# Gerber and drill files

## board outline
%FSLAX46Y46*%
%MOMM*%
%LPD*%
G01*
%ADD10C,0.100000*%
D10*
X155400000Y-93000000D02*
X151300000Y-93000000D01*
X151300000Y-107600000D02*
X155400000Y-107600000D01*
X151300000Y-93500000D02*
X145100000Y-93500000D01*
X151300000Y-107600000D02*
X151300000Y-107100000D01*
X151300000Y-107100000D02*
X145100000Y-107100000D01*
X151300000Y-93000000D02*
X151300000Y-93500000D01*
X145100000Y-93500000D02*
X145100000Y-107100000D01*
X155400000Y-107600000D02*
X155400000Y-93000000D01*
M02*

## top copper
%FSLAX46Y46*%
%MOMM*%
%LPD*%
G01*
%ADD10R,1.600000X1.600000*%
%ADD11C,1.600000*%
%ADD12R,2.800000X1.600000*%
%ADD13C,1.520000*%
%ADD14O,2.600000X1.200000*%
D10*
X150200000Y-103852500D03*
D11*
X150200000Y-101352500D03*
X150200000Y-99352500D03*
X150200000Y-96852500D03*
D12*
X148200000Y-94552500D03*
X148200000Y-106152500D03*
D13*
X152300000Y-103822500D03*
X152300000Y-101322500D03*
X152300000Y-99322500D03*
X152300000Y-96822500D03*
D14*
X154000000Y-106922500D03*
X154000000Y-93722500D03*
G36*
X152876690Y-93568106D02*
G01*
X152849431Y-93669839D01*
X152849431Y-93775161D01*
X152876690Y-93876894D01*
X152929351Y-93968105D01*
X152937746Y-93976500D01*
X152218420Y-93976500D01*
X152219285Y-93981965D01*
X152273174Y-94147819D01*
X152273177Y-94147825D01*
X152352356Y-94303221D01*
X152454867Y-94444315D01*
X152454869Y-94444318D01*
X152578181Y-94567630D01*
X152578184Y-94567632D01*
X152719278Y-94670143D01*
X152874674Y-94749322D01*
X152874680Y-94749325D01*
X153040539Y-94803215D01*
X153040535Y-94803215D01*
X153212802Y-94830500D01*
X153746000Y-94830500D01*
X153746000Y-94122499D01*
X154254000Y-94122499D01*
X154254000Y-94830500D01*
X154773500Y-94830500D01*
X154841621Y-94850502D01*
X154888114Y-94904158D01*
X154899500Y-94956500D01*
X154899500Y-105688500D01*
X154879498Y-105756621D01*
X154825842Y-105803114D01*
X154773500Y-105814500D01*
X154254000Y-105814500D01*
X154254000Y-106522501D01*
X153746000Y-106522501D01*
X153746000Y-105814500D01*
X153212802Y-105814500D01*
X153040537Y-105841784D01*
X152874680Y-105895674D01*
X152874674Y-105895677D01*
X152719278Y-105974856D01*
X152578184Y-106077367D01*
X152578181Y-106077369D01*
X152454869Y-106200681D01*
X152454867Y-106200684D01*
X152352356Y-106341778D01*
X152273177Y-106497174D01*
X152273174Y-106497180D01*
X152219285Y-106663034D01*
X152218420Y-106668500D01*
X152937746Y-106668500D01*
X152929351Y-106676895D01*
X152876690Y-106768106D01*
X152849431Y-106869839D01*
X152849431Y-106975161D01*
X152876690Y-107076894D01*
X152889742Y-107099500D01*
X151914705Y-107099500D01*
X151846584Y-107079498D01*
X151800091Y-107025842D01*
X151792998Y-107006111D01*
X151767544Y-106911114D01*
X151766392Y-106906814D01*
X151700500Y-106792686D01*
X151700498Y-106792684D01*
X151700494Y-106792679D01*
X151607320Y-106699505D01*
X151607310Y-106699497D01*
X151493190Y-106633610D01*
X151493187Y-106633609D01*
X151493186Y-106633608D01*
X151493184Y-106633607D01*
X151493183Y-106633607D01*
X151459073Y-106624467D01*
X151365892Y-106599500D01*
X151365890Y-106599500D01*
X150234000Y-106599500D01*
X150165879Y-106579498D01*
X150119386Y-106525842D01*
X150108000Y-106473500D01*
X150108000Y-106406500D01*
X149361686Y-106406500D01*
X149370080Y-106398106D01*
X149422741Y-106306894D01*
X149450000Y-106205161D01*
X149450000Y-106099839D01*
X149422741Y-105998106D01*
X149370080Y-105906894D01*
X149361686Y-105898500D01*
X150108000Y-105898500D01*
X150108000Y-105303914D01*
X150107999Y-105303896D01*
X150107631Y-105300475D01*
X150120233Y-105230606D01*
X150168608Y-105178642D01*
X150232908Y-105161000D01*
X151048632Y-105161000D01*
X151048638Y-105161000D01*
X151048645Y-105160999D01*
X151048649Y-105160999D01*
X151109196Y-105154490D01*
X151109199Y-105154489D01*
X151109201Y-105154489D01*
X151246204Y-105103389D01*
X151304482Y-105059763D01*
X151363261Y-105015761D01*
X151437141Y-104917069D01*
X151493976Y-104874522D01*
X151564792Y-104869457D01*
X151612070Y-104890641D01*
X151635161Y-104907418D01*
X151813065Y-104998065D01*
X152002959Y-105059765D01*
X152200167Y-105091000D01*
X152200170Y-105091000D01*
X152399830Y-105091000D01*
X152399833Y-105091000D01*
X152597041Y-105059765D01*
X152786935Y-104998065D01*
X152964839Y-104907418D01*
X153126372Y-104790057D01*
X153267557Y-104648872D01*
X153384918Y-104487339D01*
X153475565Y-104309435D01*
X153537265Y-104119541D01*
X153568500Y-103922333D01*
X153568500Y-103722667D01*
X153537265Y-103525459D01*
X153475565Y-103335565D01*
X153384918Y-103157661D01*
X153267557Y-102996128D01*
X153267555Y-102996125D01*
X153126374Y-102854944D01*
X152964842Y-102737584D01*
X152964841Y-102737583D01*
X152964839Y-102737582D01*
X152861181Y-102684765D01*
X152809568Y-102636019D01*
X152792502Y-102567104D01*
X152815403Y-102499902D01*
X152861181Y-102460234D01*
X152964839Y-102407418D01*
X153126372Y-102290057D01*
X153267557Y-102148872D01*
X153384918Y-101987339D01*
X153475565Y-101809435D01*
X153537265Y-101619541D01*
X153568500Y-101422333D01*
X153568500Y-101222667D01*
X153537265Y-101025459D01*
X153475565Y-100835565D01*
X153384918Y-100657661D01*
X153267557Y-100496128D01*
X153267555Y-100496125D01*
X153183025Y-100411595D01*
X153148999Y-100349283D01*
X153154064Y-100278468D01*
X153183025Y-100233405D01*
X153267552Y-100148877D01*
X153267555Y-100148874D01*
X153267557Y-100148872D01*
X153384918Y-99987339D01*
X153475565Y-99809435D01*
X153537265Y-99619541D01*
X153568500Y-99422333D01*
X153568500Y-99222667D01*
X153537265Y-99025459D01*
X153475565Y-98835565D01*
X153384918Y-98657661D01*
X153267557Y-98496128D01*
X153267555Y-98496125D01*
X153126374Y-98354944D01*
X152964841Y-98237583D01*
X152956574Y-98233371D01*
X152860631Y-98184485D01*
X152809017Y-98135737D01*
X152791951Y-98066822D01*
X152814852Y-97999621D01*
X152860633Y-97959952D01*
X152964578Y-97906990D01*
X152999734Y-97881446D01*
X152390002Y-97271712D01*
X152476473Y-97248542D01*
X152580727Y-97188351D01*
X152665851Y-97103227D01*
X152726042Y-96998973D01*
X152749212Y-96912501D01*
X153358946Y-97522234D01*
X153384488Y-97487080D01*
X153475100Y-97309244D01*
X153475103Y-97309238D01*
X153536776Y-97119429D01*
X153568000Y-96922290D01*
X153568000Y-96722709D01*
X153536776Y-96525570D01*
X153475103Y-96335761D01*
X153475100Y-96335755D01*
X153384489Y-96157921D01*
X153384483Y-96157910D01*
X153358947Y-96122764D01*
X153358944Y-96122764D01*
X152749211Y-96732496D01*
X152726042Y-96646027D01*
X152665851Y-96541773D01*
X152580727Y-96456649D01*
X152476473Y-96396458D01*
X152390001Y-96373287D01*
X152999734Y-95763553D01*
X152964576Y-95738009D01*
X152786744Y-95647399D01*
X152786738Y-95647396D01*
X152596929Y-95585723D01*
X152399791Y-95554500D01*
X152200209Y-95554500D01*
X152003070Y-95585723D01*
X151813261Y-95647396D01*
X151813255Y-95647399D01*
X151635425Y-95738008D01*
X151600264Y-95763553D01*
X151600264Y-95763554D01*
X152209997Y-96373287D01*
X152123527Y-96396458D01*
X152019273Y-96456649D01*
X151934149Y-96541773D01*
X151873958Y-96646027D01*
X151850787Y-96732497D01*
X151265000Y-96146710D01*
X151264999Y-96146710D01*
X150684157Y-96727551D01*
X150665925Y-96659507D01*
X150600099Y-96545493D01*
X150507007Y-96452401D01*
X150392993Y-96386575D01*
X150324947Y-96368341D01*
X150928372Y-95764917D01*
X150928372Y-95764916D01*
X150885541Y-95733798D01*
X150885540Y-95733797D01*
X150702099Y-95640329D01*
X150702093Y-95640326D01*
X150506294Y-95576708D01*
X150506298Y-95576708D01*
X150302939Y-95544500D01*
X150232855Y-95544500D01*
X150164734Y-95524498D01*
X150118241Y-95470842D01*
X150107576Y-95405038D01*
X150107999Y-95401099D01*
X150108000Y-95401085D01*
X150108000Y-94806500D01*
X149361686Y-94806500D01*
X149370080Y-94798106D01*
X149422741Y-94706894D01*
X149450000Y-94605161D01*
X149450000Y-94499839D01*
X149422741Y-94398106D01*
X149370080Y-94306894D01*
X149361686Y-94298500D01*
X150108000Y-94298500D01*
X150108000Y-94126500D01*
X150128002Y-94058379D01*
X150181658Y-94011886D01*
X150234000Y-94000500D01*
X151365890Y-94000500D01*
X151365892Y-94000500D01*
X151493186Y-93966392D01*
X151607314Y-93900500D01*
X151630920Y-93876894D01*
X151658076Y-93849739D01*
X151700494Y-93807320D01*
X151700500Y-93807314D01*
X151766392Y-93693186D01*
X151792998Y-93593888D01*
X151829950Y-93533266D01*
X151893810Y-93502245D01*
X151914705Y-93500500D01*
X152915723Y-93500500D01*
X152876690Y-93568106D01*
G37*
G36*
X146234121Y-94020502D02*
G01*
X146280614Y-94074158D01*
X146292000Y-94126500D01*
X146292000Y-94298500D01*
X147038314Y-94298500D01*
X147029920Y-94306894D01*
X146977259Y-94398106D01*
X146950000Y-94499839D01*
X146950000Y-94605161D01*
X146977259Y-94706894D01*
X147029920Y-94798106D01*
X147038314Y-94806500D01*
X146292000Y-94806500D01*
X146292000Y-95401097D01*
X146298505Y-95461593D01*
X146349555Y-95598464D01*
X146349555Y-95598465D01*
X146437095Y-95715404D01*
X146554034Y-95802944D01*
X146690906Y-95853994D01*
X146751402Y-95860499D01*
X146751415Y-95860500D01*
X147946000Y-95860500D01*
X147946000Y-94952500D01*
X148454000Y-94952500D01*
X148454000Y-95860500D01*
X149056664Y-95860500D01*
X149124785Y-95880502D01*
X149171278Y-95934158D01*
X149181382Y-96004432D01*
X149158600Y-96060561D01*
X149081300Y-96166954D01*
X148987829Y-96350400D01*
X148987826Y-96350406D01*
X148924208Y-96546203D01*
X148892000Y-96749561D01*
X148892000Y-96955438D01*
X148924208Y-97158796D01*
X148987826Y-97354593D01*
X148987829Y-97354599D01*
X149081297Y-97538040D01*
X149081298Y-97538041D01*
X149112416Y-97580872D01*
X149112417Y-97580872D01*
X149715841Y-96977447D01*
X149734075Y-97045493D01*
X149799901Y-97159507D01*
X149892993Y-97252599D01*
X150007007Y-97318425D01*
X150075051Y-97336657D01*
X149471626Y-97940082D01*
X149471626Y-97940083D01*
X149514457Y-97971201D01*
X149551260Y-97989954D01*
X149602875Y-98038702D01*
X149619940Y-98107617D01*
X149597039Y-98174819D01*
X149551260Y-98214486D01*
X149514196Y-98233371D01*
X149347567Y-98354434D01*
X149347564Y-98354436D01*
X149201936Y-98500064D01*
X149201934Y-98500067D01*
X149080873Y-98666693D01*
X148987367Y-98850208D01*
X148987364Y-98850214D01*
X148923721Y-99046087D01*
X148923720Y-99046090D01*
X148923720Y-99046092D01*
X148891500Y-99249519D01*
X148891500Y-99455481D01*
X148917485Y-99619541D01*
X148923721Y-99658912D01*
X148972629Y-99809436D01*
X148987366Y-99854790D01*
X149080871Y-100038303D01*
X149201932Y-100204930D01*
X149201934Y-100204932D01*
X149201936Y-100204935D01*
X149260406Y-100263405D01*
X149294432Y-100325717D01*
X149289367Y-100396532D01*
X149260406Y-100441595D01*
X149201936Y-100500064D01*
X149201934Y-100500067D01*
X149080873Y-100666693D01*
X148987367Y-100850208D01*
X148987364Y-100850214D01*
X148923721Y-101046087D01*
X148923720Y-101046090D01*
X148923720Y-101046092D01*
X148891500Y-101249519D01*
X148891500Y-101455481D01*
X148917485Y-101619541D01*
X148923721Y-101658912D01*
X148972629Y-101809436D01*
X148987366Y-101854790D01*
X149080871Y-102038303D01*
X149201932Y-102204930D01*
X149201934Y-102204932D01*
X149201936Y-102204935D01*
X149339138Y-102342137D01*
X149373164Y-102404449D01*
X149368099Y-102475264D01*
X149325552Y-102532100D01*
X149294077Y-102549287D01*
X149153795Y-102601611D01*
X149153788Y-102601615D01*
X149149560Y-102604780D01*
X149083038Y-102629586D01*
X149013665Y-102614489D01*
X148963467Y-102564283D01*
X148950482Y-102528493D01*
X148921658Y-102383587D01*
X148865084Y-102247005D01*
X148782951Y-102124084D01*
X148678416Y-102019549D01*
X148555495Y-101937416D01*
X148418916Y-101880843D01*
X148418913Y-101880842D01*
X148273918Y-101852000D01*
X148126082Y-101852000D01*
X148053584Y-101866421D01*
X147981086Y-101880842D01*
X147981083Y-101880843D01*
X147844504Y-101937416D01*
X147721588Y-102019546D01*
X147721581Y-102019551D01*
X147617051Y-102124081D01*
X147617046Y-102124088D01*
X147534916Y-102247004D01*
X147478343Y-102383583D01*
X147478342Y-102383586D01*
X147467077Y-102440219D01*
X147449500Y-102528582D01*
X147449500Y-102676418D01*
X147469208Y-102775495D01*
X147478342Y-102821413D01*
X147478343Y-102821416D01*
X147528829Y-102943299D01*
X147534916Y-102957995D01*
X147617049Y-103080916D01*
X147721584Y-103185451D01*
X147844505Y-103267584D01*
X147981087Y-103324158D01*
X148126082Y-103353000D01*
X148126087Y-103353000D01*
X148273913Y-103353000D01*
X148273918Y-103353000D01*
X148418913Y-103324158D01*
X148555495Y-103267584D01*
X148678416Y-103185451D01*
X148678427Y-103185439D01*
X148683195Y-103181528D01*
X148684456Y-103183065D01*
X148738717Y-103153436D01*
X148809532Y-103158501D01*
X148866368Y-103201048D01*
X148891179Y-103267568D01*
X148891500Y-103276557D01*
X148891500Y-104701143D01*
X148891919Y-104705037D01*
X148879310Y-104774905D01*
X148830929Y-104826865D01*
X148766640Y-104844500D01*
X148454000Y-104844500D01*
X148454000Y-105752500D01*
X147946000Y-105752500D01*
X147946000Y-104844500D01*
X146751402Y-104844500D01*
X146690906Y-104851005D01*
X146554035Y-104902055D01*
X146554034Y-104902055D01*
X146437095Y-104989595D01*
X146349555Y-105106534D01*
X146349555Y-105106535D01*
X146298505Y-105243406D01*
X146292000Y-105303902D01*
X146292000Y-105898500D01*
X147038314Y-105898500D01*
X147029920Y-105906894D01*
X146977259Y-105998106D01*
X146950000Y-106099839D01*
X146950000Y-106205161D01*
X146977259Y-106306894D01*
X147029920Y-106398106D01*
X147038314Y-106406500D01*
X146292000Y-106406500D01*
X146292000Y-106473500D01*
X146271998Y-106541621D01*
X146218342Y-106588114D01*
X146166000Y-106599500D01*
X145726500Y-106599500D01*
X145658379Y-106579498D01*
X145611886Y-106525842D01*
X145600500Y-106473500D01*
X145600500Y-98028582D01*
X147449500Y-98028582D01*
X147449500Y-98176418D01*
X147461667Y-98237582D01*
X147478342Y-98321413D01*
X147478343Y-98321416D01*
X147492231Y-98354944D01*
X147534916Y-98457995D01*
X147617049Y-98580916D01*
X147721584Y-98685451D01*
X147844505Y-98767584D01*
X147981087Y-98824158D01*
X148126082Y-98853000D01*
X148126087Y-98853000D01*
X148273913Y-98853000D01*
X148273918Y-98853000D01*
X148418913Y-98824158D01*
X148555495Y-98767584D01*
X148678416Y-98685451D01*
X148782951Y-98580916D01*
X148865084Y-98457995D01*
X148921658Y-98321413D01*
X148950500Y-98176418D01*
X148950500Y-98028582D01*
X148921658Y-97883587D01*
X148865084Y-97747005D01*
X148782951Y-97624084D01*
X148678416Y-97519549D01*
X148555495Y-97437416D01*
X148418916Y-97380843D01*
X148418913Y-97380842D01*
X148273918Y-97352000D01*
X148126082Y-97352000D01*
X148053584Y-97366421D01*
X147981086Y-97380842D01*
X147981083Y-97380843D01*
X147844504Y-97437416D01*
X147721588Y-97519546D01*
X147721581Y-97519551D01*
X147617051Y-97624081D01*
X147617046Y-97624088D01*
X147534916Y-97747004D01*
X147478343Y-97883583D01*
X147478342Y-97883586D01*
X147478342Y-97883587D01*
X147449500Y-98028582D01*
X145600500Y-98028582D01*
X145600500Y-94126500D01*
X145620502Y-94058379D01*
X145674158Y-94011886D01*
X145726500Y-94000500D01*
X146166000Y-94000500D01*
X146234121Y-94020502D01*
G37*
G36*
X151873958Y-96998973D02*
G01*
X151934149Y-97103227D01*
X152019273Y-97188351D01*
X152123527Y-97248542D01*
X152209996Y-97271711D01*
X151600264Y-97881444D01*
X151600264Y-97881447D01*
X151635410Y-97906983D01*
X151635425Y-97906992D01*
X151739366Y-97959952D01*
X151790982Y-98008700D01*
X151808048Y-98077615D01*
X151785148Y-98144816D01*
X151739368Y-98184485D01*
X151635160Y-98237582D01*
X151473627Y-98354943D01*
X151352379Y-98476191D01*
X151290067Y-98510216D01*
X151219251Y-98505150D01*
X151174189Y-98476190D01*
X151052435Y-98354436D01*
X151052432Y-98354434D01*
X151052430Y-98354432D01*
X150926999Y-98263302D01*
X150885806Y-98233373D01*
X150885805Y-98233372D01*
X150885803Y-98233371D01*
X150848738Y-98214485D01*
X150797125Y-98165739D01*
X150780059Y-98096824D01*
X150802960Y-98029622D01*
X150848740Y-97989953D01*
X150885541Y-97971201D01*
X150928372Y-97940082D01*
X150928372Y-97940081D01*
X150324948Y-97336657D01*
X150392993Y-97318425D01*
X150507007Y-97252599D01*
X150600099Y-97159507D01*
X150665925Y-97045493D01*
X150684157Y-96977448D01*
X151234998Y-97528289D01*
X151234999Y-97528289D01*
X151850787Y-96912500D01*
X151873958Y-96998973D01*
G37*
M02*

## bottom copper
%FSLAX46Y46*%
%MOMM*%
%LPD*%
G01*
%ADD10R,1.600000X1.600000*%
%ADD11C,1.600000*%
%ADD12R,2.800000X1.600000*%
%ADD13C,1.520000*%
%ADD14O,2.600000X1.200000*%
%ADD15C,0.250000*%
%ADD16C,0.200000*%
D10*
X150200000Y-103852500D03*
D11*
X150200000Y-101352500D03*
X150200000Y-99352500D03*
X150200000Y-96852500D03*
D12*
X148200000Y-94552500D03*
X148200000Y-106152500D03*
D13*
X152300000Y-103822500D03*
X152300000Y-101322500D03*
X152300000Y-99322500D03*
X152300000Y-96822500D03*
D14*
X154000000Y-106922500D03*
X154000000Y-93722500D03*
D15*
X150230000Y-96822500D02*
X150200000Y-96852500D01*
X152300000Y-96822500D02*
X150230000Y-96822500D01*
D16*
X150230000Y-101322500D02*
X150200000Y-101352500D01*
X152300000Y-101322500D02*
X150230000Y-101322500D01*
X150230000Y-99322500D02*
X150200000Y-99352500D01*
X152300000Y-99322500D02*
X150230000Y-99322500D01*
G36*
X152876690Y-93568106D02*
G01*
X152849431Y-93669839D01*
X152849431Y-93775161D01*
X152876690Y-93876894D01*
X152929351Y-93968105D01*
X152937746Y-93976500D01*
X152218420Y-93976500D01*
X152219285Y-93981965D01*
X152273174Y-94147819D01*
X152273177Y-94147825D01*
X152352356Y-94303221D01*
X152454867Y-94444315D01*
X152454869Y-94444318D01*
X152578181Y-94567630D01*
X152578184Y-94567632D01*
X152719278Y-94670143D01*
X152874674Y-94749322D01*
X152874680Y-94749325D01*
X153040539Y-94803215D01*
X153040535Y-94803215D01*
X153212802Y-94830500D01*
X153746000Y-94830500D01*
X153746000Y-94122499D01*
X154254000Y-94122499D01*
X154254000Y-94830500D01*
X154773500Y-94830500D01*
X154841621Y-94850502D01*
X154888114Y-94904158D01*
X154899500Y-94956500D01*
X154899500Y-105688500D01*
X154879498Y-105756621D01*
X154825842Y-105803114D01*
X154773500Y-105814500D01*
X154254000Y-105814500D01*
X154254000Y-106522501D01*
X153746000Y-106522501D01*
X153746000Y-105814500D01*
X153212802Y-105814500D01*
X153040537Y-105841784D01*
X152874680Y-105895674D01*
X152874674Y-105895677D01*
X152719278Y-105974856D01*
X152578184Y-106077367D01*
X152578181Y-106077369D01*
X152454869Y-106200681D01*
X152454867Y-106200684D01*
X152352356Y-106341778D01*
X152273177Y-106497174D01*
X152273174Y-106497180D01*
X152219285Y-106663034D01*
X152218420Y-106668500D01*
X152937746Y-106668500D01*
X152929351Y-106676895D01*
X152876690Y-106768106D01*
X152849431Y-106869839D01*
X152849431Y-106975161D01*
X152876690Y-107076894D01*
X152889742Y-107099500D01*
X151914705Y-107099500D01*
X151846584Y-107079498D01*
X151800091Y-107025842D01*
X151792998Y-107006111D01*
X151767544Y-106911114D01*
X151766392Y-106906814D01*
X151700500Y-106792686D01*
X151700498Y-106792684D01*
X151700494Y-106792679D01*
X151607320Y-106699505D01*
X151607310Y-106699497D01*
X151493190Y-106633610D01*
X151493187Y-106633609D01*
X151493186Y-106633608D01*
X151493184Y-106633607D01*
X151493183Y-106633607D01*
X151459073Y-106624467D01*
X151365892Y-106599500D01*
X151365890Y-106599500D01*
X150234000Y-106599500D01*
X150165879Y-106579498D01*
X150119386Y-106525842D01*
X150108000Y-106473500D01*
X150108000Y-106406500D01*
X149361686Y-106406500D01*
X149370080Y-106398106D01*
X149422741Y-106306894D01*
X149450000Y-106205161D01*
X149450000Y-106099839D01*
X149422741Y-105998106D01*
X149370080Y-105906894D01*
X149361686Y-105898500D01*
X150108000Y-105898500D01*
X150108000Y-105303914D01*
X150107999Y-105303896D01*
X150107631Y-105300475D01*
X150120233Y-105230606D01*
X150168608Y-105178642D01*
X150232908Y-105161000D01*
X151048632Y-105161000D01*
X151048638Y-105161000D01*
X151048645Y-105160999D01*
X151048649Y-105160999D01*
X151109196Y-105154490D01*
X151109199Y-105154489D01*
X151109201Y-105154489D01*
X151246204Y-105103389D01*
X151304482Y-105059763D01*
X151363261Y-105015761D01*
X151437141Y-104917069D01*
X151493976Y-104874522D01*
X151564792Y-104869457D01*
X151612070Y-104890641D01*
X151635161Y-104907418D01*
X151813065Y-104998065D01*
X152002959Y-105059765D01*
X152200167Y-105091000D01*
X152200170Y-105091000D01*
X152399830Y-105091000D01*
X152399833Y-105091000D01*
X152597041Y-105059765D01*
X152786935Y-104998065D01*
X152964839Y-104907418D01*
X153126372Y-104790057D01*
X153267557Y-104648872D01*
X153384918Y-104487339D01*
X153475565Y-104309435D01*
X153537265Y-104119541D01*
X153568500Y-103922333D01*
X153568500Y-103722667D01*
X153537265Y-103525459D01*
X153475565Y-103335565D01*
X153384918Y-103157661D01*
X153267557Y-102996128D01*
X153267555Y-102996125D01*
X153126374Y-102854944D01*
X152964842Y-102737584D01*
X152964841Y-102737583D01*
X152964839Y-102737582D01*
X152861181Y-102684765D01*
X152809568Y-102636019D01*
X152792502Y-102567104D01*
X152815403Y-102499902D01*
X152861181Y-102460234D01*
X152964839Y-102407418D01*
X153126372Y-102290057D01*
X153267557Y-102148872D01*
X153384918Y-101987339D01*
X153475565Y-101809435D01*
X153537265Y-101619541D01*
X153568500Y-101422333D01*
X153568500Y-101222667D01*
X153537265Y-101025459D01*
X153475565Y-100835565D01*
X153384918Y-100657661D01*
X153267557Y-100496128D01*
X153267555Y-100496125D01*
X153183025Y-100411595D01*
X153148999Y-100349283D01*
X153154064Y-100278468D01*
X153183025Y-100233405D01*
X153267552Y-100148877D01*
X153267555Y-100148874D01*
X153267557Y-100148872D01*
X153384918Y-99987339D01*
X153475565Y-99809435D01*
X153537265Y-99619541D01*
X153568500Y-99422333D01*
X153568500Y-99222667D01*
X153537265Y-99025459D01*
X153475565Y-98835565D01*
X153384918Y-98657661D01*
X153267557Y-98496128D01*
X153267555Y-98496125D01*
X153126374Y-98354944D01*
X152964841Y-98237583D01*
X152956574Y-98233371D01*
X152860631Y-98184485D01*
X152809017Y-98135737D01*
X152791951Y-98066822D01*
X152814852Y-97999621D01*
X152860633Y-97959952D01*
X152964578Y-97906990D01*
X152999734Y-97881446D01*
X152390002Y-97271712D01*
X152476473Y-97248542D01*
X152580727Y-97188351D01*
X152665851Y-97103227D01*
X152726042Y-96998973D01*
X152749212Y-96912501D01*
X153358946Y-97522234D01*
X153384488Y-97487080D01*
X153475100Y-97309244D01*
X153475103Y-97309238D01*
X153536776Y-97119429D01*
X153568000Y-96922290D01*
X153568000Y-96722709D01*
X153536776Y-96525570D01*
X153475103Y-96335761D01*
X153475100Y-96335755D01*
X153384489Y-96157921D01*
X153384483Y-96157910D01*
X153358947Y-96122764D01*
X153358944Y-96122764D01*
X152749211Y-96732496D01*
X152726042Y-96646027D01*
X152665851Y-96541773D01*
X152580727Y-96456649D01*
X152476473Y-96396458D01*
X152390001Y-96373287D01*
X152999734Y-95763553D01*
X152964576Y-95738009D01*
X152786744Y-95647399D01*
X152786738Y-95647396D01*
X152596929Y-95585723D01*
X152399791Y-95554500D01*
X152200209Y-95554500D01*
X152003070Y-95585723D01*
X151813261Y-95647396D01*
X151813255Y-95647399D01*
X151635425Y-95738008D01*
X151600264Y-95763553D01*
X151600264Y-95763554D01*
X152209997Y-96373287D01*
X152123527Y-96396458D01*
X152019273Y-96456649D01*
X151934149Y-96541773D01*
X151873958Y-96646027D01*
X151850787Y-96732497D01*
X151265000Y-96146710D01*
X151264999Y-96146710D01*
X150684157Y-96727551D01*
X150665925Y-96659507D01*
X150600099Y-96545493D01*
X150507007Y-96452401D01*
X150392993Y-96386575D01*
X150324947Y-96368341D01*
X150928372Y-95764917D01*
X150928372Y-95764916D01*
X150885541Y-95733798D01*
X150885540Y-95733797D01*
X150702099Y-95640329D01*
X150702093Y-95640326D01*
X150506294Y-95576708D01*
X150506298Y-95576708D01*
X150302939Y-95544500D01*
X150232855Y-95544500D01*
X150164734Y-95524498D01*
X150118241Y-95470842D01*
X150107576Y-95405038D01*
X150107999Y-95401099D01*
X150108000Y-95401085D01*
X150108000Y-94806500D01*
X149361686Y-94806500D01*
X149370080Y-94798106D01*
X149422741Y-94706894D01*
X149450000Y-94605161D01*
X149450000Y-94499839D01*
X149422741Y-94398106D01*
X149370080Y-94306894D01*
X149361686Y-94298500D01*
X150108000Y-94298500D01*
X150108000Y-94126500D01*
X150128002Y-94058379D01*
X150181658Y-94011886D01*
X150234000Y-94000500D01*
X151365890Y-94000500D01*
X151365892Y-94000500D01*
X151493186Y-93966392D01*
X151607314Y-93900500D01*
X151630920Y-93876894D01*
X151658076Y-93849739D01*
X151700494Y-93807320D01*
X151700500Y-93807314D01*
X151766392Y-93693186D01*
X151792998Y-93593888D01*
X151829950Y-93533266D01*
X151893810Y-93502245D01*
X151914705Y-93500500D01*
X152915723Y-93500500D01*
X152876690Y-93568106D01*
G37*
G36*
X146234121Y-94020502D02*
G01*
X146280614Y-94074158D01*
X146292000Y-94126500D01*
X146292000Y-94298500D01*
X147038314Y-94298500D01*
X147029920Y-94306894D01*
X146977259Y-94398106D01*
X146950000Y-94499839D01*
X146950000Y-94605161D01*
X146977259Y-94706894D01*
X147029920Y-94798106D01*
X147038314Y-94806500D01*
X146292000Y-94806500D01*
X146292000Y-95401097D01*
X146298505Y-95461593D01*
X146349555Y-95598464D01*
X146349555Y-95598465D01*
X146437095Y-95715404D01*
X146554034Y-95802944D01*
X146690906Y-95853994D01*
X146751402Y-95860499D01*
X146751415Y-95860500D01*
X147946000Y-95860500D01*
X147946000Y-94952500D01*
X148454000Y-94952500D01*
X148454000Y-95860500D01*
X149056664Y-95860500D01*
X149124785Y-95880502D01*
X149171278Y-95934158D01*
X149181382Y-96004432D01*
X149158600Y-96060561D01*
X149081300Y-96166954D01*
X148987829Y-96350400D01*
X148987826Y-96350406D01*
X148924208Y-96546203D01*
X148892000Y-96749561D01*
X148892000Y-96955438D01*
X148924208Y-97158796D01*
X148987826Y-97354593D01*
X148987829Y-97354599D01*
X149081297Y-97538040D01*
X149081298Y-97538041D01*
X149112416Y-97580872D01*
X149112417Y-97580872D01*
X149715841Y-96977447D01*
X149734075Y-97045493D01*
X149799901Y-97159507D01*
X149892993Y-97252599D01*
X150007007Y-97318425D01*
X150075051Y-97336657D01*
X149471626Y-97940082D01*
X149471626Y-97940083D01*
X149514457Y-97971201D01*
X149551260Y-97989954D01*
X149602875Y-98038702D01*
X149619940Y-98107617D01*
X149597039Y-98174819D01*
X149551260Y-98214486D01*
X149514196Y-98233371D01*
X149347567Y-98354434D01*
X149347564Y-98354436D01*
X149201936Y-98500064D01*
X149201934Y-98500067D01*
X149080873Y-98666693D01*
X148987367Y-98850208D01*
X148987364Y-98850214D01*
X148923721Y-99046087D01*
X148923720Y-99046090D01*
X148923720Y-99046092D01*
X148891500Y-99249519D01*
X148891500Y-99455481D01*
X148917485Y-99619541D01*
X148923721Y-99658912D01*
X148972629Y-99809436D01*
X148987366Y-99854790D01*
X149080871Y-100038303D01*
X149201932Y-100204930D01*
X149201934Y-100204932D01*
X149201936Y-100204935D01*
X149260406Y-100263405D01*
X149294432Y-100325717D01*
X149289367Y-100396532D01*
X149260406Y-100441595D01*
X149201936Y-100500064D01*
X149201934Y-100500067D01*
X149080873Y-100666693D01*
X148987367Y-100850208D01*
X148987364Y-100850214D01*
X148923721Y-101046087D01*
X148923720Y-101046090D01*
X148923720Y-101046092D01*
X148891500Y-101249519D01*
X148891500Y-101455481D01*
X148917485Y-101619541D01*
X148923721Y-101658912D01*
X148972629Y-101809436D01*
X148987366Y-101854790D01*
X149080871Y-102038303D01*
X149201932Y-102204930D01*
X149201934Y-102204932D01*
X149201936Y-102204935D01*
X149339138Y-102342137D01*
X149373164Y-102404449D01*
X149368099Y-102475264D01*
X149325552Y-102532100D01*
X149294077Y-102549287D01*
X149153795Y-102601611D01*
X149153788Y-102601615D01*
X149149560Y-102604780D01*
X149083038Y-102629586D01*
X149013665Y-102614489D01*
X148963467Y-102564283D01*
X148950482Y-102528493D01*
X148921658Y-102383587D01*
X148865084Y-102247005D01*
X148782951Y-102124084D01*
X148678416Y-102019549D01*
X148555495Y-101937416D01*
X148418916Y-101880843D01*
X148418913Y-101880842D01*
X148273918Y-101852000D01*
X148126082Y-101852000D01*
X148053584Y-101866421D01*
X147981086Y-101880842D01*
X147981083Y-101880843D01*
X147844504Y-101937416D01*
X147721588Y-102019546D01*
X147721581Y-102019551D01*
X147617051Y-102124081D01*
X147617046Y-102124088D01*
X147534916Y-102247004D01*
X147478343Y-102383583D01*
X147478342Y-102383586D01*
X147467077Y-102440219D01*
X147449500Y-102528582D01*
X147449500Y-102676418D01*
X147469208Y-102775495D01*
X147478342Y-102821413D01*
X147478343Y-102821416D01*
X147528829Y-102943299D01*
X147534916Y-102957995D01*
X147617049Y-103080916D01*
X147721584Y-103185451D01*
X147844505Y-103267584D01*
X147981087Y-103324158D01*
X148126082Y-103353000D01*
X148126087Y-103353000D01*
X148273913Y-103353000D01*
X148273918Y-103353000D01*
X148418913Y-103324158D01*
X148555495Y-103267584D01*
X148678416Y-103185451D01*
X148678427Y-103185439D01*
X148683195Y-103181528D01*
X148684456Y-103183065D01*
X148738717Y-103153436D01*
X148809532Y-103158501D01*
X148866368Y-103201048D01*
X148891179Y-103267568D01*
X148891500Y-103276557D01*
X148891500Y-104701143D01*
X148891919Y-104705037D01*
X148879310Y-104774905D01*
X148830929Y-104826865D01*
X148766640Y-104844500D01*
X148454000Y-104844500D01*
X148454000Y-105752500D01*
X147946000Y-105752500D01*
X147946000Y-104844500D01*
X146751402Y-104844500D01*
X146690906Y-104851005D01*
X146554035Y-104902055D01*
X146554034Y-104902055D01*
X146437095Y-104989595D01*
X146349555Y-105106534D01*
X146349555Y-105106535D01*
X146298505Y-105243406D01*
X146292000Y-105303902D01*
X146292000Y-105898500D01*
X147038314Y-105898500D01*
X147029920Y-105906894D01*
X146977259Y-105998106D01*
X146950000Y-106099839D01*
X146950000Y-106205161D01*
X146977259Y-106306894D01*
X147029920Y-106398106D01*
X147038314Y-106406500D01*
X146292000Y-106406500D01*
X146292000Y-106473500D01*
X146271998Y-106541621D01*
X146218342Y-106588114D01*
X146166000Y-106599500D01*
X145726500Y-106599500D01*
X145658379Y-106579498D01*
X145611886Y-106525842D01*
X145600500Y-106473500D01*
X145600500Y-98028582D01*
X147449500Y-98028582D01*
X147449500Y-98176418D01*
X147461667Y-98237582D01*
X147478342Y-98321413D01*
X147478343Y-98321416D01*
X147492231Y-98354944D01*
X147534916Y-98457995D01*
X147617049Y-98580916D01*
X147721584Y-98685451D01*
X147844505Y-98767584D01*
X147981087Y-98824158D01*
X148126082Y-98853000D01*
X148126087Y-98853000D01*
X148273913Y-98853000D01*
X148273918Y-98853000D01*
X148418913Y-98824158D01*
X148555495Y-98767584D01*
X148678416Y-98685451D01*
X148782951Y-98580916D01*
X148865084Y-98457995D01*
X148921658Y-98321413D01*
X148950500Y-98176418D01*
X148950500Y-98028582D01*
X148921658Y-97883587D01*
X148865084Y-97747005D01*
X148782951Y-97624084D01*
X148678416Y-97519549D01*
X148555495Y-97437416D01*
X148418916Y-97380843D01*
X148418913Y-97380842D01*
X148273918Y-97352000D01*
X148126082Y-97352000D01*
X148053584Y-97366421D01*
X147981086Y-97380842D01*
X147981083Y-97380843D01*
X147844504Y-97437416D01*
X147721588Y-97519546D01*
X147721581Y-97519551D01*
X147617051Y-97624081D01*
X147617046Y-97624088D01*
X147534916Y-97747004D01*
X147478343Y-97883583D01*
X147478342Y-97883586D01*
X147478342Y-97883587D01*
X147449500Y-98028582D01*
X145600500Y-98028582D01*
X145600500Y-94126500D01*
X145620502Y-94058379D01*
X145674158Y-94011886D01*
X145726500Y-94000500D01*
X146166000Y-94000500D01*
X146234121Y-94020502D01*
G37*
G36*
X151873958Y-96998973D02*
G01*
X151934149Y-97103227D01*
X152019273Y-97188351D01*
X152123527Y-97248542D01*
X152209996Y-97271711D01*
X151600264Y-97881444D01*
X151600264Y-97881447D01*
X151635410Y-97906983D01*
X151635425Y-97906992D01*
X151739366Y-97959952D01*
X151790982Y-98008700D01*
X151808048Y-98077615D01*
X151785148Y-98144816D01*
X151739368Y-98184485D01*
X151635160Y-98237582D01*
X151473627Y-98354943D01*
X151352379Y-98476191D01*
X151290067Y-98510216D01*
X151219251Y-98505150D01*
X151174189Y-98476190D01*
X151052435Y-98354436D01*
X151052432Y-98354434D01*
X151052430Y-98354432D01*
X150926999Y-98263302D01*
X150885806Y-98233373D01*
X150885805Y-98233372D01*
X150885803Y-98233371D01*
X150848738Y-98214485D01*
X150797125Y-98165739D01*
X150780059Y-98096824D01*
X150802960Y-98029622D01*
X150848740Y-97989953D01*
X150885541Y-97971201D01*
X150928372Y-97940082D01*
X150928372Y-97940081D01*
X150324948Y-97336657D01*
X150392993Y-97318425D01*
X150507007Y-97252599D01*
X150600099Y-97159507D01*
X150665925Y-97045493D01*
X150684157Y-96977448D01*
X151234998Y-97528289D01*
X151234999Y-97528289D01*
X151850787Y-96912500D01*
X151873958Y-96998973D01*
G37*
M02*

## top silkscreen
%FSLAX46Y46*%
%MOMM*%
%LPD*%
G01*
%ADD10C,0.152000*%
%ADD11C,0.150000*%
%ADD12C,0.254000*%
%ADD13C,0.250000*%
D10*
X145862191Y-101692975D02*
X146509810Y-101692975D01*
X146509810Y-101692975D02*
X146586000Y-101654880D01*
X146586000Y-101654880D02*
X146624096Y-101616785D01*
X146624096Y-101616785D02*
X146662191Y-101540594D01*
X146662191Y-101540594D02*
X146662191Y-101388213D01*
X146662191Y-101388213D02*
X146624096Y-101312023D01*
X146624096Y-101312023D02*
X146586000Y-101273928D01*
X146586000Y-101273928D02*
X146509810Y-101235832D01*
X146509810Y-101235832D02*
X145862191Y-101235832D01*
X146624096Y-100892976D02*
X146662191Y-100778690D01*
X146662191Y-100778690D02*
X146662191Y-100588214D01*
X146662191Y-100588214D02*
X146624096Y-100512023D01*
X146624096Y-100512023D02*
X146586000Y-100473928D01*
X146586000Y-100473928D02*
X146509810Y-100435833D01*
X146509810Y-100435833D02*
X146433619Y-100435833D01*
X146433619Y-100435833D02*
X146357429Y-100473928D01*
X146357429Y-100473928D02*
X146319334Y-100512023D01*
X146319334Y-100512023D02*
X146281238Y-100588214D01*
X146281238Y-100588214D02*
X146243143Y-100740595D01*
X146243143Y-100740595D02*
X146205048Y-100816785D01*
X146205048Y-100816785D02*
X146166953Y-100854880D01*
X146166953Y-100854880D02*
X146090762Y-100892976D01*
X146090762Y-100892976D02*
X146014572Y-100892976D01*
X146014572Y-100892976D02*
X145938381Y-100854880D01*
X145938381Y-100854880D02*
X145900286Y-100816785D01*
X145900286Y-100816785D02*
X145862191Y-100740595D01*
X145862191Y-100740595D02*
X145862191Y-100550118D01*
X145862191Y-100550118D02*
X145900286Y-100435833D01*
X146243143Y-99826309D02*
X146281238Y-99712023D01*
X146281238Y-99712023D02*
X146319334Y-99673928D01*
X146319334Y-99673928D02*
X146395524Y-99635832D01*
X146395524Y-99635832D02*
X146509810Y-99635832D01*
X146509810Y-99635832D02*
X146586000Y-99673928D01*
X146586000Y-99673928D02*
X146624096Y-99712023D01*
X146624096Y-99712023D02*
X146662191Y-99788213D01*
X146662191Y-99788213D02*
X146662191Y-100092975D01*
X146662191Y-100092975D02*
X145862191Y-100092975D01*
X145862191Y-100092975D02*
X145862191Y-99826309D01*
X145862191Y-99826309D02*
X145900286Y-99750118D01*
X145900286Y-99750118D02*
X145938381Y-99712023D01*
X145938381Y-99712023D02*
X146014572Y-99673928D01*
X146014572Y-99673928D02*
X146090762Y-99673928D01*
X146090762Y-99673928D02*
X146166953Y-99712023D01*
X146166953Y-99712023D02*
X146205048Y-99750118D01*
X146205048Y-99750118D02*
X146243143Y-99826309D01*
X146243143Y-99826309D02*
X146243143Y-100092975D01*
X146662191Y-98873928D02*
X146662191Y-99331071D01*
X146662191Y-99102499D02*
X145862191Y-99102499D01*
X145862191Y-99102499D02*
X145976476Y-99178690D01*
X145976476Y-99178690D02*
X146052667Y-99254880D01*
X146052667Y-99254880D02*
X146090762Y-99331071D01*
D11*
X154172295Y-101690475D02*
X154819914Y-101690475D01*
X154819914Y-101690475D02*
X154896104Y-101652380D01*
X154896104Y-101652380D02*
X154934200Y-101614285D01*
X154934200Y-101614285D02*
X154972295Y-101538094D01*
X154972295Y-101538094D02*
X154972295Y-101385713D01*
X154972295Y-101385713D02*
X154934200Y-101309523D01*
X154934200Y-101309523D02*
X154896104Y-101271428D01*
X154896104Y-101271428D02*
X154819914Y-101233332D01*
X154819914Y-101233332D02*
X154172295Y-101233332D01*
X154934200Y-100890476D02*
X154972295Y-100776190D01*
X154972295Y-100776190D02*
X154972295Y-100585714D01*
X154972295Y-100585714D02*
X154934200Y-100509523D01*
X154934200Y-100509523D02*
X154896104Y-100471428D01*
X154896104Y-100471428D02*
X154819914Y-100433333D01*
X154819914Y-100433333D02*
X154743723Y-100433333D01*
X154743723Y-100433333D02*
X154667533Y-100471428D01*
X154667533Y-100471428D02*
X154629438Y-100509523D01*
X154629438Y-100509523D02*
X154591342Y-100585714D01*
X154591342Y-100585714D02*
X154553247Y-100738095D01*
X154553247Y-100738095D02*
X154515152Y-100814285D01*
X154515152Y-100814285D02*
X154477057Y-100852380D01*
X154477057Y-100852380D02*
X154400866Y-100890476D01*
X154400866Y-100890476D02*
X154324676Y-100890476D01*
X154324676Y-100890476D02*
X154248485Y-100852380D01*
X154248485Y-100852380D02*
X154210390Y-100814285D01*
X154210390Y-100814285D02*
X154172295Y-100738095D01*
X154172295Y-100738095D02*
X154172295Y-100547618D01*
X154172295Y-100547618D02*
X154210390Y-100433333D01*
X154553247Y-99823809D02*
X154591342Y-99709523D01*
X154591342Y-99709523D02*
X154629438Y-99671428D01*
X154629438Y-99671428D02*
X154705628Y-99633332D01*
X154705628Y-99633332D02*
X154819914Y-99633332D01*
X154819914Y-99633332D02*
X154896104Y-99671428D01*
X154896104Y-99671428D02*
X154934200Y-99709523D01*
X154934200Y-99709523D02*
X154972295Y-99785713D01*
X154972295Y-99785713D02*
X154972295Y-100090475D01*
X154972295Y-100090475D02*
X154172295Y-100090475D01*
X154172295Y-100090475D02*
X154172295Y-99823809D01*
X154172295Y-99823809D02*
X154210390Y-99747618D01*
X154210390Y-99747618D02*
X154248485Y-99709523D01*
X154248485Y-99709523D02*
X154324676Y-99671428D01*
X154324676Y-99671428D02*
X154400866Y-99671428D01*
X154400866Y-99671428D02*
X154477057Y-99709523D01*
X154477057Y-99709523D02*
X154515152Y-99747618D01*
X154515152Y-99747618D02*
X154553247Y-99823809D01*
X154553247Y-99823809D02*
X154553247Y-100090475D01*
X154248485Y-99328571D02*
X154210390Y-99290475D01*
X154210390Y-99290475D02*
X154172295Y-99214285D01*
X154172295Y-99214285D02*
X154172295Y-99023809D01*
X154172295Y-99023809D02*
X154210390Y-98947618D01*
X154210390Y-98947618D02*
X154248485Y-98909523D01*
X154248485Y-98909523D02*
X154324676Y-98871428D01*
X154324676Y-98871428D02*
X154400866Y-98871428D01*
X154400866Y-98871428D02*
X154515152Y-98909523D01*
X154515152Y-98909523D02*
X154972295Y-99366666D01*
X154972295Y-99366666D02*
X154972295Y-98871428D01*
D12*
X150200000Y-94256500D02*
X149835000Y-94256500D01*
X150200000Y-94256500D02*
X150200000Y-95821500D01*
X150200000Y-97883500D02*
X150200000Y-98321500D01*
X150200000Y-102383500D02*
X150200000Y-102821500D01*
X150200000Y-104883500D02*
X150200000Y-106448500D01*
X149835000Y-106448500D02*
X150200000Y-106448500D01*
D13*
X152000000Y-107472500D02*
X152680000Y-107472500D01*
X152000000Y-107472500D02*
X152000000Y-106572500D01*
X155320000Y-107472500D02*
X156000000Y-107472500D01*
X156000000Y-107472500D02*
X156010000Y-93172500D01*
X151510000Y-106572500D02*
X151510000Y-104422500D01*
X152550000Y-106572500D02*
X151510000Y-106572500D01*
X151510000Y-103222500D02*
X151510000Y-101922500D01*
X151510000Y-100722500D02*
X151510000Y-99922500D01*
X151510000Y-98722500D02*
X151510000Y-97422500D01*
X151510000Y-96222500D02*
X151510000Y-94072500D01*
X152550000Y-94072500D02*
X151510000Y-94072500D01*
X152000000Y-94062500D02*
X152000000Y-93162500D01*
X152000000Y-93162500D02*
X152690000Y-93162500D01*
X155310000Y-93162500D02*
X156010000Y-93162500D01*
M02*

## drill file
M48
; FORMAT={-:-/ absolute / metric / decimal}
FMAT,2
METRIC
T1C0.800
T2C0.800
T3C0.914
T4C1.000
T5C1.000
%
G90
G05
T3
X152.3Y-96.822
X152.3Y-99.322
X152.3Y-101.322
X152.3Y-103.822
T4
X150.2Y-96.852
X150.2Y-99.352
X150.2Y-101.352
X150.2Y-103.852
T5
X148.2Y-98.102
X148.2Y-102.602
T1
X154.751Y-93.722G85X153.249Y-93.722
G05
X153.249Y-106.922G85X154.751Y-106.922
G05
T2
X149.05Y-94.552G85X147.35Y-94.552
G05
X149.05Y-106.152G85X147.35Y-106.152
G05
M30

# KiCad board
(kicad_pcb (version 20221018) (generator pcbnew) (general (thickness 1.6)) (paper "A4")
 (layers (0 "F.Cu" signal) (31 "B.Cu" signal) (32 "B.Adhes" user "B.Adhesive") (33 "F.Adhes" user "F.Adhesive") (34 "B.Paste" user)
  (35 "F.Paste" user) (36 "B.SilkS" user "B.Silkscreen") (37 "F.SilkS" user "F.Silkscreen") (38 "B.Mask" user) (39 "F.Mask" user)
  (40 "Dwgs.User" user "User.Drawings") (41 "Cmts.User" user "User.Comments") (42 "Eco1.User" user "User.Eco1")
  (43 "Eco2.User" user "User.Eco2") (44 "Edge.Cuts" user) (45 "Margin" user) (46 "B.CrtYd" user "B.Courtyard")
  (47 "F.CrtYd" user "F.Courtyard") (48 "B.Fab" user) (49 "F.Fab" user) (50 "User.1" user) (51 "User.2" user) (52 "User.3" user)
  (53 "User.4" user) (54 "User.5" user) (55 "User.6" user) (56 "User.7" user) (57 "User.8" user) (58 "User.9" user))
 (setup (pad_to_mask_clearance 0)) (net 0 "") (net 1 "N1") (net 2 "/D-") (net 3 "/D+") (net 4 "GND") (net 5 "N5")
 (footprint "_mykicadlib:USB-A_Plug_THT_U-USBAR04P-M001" (layer "F.Cu") (at 149 100.3525 -90)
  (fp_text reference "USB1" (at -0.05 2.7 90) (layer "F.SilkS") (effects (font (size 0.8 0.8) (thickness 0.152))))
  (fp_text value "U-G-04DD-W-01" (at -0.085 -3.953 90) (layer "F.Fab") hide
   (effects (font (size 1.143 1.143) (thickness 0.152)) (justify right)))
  (fp_line (start -6.096 -1.2) (end -6.096 -0.835) (stroke (width 0.254) (type solid)) (layer "F.SilkS"))
  (fp_line (start -6.096 -1.2) (end -4.531 -1.2) (stroke (width 0.254) (type solid)) (layer "F.SilkS"))
  (fp_line (start -2.469 -1.2) (end -2.031 -1.2) (stroke (width 0.254) (type solid)) (layer "F.SilkS"))
  (fp_line (start 2.031 -1.2) (end 2.469 -1.2) (stroke (width 0.254) (type solid)) (layer "F.SilkS"))
  (fp_line (start 4.531 -1.2) (end 6.096 -1.2) (stroke (width 0.254) (type solid)) (layer "F.SilkS"))
  (fp_line (start 6.096 -0.835) (end 6.096 -1.2) (stroke (width 0.254) (type solid)) (layer "F.SilkS"))
  (pad "" np_thru_hole circle (at -2.25 0.8 270) (size 1 1) (drill 1) (layers "*.Cu" "*.Mask"))
  (pad "" np_thru_hole circle (at 2.25 0.8 270) (size 1 1) (drill 1) (layers "*.Cu" "*.Mask"))
  (pad "1" thru_hole rect (at 3.5 -1.2 270) (size 1.6 1.6) (drill 1) (layers "*.Cu" "*.Mask") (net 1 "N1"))
  (pad "2" thru_hole circle (at 1 -1.2 270) (size 1.6 1.6) (drill 1) (layers "*.Cu" "*.Mask") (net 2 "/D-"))
  (pad "3" thru_hole circle (at -1 -1.2 270) (size 1.6 1.6) (drill 1) (layers "*.Cu" "*.Mask") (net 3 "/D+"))
  (pad "4" thru_hole circle (at -3.5 -1.2 270) (size 1.6 1.6) (drill 1) (layers "*.Cu" "*.Mask") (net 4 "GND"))
  (pad "5" thru_hole rect (at -5.8 0.8 270) (size 1.6 2.8) (drill oval 0.8 2.5) (layers "*.Cu" "*.Mask") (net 4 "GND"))
  (pad "5" thru_hole rect (at 5.8 0.8 270) (size 1.6 2.8) (drill oval 0.8 2.5) (layers "*.Cu" "*.Mask") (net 4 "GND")))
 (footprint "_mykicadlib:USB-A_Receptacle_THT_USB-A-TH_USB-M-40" (layer "F.Cu") (at 153.41 100.3225 90)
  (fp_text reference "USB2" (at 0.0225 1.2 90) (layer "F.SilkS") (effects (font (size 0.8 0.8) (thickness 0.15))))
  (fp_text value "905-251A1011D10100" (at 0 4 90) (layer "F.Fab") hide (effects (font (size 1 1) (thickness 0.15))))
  (fp_line (start -7.15 -1.41) (end -7.15 -0.73) (stroke (width 0.25) (type solid)) (layer "F.SilkS"))
  (fp_line (start -7.15 -1.41) (end -6.25 -1.41) (stroke (width 0.25) (type solid)) (layer "F.SilkS"))
  (fp_line (start -7.15 1.91) (end -7.15 2.59) (stroke (width 0.25) (type solid)) (layer "F.SilkS"))
  (fp_line (start -7.15 2.59) (end 7.15 2.6) (stroke (width 0.25) (type solid)) (layer "F.SilkS"))
  (fp_line (start -6.25 -1.9) (end -4.1 -1.9) (stroke (width 0.25) (type solid)) (layer "F.SilkS"))
  (fp_line (start -6.25 -0.86) (end -6.25 -1.9) (stroke (width 0.25) (type solid)) (layer "F.SilkS"))
  (fp_line (start -2.9 -1.9) (end -1.6 -1.9) (stroke (width 0.25) (type solid)) (layer "F.SilkS"))
  (fp_line (start -0.4 -1.9) (end 0.4 -1.9) (stroke (width 0.25) (type solid)) (layer "F.SilkS"))
  (fp_line (start 1.6 -1.9) (end 2.9 -1.9) (stroke (width 0.25) (type solid)) (layer "F.SilkS"))
  (fp_line (start 4.1 -1.9) (end 6.25 -1.9) (stroke (width 0.25) (type solid)) (layer "F.SilkS"))
  (fp_line (start 6.25 -0.86) (end 6.25 -1.9) (stroke (width 0.25) (type solid)) (layer "F.SilkS"))
  (fp_line (start 6.26 -1.41) (end 7.16 -1.41) (stroke (width 0.25) (type solid)) (layer "F.SilkS"))
  (fp_line (start 7.16 -1.41) (end 7.16 -0.72) (stroke (width 0.25) (type solid)) (layer "F.SilkS"))
  (fp_line (start 7.16 1.9) (end 7.16 2.6) (stroke (width 0.25) (type solid)) (layer "F.SilkS"))
  (pad "1" thru_hole circle (at -3.5 -1.11 90) (size 1.52 1.52) (drill 0.9144) (layers "*.Cu" "*.Paste" "*.Mask") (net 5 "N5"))
  (pad "2" thru_hole circle (at -1 -1.11 90) (size 1.52 1.52) (drill 0.9144) (layers "*.Cu" "*.Paste" "*.Mask") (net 2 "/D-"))
  (pad "3" thru_hole circle (at 1 -1.11 90) (size 1.52 1.52) (drill 0.9144) (layers "*.Cu" "*.Paste" "*.Mask") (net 3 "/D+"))
  (pad "4" thru_hole circle (at 3.5 -1.11 90) (size 1.52 1.52) (drill 0.9144) (layers "*.Cu" "*.Paste" "*.Mask") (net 4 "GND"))
  (pad "5" thru_hole oval (at -6.6 0.59) (size 2.6 1.2) (drill oval 2.301138 0.799998) (layers "*.Cu" "*.Paste" "*.Mask") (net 4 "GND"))
  (pad "5" thru_hole oval (at 6.6 0.59 180) (size 2.6 1.2) (drill oval 2.301138 0.799998) (layers "*.Cu" "*.Paste" "*.Mask") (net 4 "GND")))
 (gr_line (start 155.4 93) (end 151.3 93) (stroke (width 0.1) (type solid)) (layer "Edge.Cuts"))
 (gr_line (start 151.3 107.6) (end 155.4 107.6) (stroke (width 0.1) (type solid)) (layer "Edge.Cuts"))
 (gr_line (start 151.3 93.5) (end 145.1 93.5) (stroke (width 0.1) (type solid)) (layer "Edge.Cuts"))
 (gr_line (start 151.3 107.6) (end 151.3 107.1) (stroke (width 0.1) (type solid)) (layer "Edge.Cuts"))
 (gr_line (start 151.3 107.1) (end 145.1 107.1) (stroke (width 0.1) (type solid)) (layer "Edge.Cuts"))
 (gr_line (start 151.3 93) (end 151.3 93.5) (stroke (width 0.1) (type solid)) (layer "Edge.Cuts"))
 (gr_line (start 145.1 93.5) (end 145.1 107.1) (stroke (width 0.1) (type solid)) (layer "Edge.Cuts"))
 (gr_line (start 155.4 107.6) (end 155.4 93) (stroke (width 0.1) (type solid)) (layer "Edge.Cuts"))
 (segment (start 150.23 96.8225) (end 150.2 96.8525) (width 0.25) (layer "B.Cu") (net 4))
 (segment (start 152.3 96.8225) (end 150.23 96.8225) (width 0.25) (layer "B.Cu") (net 4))
 (segment (start 150.23 101.3225) (end 150.2 101.3525) (width 0.2) (layer "B.Cu") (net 2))
 (segment (start 152.3 101.3225) (end 150.23 101.3225) (width 0.2) (layer "B.Cu") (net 2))
 (segment (start 150.23 99.3225) (end 150.2 99.3525) (width 0.2) (layer "B.Cu") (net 3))
 (segment (start 152.3 99.3225) (end 150.23 99.3225) (width 0.2) (layer "B.Cu") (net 3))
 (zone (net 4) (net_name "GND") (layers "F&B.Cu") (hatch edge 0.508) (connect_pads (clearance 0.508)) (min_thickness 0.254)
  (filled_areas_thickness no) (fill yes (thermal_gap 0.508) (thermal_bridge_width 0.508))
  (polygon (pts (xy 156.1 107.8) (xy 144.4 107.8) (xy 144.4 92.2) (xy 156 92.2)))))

